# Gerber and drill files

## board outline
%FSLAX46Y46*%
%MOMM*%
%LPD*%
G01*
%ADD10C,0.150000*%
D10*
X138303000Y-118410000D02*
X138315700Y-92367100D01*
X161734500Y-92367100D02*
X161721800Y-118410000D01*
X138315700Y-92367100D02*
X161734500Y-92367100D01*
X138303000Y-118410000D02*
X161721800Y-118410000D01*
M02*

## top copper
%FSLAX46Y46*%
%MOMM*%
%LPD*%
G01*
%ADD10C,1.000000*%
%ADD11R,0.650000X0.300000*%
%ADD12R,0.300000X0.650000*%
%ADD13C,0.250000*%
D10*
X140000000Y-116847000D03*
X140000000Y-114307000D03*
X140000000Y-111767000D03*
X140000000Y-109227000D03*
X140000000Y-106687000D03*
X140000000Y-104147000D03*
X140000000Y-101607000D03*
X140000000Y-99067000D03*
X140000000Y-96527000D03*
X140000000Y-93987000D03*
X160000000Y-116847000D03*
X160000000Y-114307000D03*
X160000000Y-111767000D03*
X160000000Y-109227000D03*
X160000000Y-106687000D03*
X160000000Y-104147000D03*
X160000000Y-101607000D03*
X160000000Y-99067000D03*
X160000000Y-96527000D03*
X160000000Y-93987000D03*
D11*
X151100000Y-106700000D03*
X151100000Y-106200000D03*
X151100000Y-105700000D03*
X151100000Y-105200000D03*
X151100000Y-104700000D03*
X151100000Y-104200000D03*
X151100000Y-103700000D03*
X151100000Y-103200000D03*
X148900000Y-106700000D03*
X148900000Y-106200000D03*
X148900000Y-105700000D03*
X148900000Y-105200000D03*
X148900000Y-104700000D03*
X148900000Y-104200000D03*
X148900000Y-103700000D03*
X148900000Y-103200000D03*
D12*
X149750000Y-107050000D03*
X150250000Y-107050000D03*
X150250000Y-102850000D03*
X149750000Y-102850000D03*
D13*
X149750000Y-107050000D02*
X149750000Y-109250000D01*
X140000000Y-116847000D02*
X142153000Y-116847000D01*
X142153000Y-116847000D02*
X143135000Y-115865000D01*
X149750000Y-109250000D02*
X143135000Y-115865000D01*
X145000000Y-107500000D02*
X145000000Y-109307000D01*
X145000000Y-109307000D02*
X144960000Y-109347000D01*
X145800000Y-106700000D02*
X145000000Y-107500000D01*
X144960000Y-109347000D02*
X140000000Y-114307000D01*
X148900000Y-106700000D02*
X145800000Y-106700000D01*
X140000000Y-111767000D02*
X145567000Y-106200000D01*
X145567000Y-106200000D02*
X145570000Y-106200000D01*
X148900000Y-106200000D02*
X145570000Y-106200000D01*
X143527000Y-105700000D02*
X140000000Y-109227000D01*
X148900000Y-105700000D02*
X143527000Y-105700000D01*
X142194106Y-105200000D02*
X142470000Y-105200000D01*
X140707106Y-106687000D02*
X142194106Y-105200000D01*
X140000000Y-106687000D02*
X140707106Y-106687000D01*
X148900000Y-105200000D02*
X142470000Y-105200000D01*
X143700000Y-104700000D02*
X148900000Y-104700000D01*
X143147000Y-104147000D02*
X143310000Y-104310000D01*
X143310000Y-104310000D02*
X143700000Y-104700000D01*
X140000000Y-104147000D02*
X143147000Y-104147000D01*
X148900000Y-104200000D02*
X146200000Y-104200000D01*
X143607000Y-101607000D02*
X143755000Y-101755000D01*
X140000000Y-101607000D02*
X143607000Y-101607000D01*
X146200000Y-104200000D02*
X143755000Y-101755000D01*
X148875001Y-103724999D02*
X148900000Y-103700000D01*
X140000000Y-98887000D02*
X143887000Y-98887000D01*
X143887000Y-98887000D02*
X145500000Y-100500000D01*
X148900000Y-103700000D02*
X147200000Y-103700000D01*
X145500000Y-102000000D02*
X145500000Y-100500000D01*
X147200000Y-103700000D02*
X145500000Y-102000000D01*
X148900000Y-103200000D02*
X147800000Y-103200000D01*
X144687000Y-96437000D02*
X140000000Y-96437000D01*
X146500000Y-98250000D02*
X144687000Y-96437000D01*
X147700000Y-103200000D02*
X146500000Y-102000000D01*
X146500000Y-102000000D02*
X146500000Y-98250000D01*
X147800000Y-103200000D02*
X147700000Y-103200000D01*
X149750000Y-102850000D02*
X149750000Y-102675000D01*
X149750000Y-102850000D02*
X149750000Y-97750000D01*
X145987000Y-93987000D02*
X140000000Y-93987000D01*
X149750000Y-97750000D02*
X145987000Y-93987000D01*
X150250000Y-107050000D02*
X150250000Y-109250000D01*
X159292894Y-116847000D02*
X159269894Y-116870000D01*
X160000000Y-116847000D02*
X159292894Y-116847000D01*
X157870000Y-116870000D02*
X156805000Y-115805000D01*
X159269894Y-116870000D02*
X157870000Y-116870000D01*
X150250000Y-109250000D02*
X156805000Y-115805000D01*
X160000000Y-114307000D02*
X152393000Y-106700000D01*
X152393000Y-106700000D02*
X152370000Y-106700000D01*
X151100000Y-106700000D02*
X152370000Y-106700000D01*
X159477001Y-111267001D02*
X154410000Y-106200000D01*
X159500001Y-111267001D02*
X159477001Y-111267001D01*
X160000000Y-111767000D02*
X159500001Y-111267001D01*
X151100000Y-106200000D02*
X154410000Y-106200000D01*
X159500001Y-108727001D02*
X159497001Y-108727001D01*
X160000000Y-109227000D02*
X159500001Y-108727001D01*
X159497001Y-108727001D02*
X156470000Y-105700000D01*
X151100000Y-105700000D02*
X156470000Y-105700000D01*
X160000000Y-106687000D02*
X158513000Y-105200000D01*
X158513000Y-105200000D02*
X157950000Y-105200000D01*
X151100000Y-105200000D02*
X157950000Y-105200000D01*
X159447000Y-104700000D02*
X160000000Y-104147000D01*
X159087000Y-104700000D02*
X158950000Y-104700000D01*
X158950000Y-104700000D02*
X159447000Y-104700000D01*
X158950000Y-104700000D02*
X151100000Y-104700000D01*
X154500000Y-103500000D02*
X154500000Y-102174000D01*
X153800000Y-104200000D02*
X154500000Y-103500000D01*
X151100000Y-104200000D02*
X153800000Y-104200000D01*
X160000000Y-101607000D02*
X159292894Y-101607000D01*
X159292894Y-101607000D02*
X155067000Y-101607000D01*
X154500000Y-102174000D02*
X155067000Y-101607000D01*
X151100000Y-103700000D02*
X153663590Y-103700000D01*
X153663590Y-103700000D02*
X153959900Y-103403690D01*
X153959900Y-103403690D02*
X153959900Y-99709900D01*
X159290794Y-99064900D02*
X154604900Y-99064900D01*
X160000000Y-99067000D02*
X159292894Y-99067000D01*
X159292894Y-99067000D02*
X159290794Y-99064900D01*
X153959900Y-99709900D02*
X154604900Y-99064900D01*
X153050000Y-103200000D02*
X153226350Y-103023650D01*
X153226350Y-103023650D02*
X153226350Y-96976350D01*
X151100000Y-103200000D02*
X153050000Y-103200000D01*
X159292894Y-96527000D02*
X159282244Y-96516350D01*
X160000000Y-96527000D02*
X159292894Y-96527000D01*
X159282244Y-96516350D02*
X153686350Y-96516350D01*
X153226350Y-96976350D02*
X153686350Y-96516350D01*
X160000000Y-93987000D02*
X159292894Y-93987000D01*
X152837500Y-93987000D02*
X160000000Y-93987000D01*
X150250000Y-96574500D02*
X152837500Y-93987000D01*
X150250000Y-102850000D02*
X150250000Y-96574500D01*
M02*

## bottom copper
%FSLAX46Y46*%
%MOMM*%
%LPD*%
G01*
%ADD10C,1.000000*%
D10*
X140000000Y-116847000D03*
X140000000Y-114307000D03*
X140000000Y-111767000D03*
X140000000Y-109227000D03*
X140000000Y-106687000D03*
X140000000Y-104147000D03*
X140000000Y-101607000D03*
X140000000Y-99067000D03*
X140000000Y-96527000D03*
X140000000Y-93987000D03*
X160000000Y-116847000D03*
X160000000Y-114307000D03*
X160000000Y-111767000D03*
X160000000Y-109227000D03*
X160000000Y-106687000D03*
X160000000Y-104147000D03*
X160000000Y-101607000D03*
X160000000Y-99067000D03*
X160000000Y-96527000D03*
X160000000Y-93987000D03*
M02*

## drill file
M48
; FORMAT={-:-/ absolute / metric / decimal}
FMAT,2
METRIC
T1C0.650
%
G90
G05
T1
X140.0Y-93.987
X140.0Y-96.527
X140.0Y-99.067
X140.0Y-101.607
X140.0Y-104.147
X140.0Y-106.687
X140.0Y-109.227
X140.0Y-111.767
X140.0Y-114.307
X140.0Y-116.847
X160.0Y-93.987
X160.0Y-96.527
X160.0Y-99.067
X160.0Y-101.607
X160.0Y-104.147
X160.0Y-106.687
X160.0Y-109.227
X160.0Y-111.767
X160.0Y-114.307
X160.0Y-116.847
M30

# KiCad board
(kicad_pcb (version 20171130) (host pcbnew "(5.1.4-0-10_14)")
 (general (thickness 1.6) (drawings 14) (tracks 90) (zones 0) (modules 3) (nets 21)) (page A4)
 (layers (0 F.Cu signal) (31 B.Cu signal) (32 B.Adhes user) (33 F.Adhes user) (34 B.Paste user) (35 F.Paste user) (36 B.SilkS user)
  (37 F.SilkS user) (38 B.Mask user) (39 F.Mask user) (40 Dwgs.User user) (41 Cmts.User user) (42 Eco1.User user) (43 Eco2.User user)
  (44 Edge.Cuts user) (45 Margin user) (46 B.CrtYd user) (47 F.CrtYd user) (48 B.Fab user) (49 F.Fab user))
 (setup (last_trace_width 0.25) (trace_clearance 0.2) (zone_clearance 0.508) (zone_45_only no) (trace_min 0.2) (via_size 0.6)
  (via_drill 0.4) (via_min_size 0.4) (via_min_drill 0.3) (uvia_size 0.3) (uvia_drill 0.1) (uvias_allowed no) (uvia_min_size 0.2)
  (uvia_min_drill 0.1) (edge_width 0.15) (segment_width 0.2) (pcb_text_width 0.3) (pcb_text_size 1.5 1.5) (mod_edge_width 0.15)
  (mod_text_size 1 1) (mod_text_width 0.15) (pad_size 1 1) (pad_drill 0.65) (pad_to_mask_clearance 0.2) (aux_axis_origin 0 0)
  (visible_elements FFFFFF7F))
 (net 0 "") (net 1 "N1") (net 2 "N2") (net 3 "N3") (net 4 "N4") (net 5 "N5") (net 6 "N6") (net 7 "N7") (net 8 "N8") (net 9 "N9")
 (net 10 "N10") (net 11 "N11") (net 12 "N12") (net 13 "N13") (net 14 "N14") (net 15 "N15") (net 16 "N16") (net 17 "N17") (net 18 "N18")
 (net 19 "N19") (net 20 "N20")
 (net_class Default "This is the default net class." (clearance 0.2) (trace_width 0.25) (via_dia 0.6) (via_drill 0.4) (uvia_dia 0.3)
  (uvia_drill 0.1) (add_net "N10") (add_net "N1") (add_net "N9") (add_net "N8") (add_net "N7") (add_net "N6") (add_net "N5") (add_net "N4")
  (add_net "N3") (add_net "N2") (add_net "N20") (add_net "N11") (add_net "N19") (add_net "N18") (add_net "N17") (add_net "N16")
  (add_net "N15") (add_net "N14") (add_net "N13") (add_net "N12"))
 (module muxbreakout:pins (layer F.Cu) (at 140 105)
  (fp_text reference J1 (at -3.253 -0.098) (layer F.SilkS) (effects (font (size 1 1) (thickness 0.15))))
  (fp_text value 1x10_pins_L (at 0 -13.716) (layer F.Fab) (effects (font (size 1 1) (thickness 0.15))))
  (pad 10 thru_hole circle (at 0 11.847) (size 1 1) (drill 0.65) (layers *.Cu *.Mask) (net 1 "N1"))
  (pad 9 thru_hole circle (at 0 9.307) (size 1 1) (drill 0.65) (layers *.Cu *.Mask) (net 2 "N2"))
  (pad 8 thru_hole circle (at 0 6.767) (size 1 1) (drill 0.65) (layers *.Cu *.Mask) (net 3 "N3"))
  (pad 7 thru_hole circle (at 0 4.227) (size 1 1) (drill 0.65) (layers *.Cu *.Mask) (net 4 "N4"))
  (pad 6 thru_hole circle (at 0 1.687) (size 1 1) (drill 0.65) (layers *.Cu *.Mask) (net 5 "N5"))
  (pad 5 thru_hole circle (at 0 -0.853) (size 1 1) (drill 0.65) (layers *.Cu *.Mask) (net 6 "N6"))
  (pad 4 thru_hole circle (at 0 -3.393) (size 1 1) (drill 0.65) (layers *.Cu *.Mask) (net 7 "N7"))
  (pad 3 thru_hole circle (at 0 -5.933) (size 1 1) (drill 0.65) (layers *.Cu *.Mask) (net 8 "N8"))
  (pad 2 thru_hole circle (at 0 -8.473) (size 1 1) (drill 0.65) (layers *.Cu *.Mask) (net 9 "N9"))
  (pad 1 thru_hole circle (at 0 -11.013) (size 1 1) (drill 0.65) (layers *.Cu *.Mask) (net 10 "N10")))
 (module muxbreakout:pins (layer F.Cu) (at 160 105)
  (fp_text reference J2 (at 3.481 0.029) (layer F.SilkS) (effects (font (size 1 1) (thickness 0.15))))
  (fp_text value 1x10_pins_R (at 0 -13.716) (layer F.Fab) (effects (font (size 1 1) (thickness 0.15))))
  (pad 10 thru_hole circle (at 0 11.847) (size 1 1) (drill 0.65) (layers *.Cu *.Mask) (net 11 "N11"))
  (pad 9 thru_hole circle (at 0 9.307) (size 1 1) (drill 0.65) (layers *.Cu *.Mask) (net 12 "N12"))
  (pad 8 thru_hole circle (at 0 6.767) (size 1 1) (drill 0.65) (layers *.Cu *.Mask) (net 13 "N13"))
  (pad 7 thru_hole circle (at 0 4.227) (size 1 1) (drill 0.65) (layers *.Cu *.Mask) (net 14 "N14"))
  (pad 6 thru_hole circle (at 0 1.687) (size 1 1) (drill 0.65) (layers *.Cu *.Mask) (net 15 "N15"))
  (pad 5 thru_hole circle (at 0 -0.853) (size 1 1) (drill 0.65) (layers *.Cu *.Mask) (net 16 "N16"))
  (pad 4 thru_hole circle (at 0 -3.393) (size 1 1) (drill 0.65) (layers *.Cu *.Mask) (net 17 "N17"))
  (pad 3 thru_hole circle (at 0 -5.933) (size 1 1) (drill 0.65) (layers *.Cu *.Mask) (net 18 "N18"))
  (pad 2 thru_hole circle (at 0 -8.473) (size 1 1) (drill 0.65) (layers *.Cu *.Mask) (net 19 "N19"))
  (pad 1 thru_hole circle (at 0 -11.013) (size 1 1) (drill 0.65) (layers *.Cu *.Mask) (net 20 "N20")))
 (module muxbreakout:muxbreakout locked (layer F.Cu) (at 150 105)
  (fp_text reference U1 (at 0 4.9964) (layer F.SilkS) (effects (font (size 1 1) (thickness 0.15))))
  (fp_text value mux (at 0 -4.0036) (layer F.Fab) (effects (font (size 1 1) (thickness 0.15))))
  (pad 12 smd rect (at 1.1 1.7) (size 0.65 0.3) (layers F.Cu F.Paste F.Mask) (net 12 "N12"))
  (pad 13 smd rect (at 1.1 1.2) (size 0.65 0.3) (layers F.Cu F.Paste F.Mask) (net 13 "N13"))
  (pad 14 smd rect (at 1.1 0.7) (size 0.65 0.3) (layers F.Cu F.Paste F.Mask) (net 14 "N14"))
  (pad 15 smd rect (at 1.1 0.2) (size 0.65 0.3) (layers F.Cu F.Paste F.Mask) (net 15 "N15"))
  (pad 16 smd rect (at 1.1 -0.3) (size 0.65 0.3) (layers F.Cu F.Paste F.Mask) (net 16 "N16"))
  (pad 17 smd rect (at 1.1 -0.8) (size 0.65 0.3) (layers F.Cu F.Paste F.Mask) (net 17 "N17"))
  (pad 18 smd rect (at 1.1 -1.3) (size 0.65 0.3) (layers F.Cu F.Paste F.Mask) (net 18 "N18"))
  (pad 19 smd rect (at 1.1 -1.8) (size 0.65 0.3) (layers F.Cu F.Paste F.Mask) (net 19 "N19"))
  (pad 9 smd rect (at -1.1 1.7) (size 0.65 0.3) (layers F.Cu F.Paste F.Mask) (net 2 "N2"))
  (pad 8 smd rect (at -1.1 1.2) (size 0.65 0.3) (layers F.Cu F.Paste F.Mask) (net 3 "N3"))
  (pad 7 smd rect (at -1.1 0.7) (size 0.65 0.3) (layers F.Cu F.Paste F.Mask) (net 4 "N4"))
  (pad 6 smd rect (at -1.1 0.2) (size 0.65 0.3) (layers F.Cu F.Paste F.Mask) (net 5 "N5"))
  (pad 5 smd rect (at -1.1 -0.3) (size 0.65 0.3) (layers F.Cu F.Paste F.Mask) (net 6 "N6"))
  (pad 4 smd rect (at -1.1 -0.8) (size 0.65 0.3) (layers F.Cu F.Paste F.Mask) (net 7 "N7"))
  (pad 3 smd rect (at -1.1 -1.3) (size 0.65 0.3) (layers F.Cu F.Paste F.Mask) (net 8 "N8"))
  (pad 2 smd rect (at -1.1 -1.8) (size 0.65 0.3) (layers F.Cu F.Paste F.Mask) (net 9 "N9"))
  (pad 10 smd rect (at -0.25 2.05) (size 0.3 0.65) (layers F.Cu F.Paste F.Mask) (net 1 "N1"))
  (pad 11 smd rect (at 0.25 2.05) (size 0.3 0.65) (layers F.Cu F.Paste F.Mask) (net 11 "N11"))
  (pad 20 smd rect (at 0.25 -2.15) (size 0.3 0.65) (layers F.Cu F.Paste F.Mask) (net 20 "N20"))
  (pad 1 smd rect (at -0.25 -2.15) (size 0.3 0.65) (layers F.Cu F.Paste F.Mask) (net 10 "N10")))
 (gr_line (start 138.303 118.41) (end 138.3157 92.3671) (layer Edge.Cuts) (width 0.15))
 (gr_line (start 161.7345 92.3671) (end 161.7218 118.41) (layer Edge.Cuts) (width 0.15))
 (gr_line (start 138.3157 92.3671) (end 161.7345 92.3671) (layer Edge.Cuts) (width 0.15))
 (gr_line (start 138.303 118.41) (end 161.7218 118.41) (layer Edge.Cuts) (width 0.15))
 (segment (start 149.75 107.05) (end 149.75 109.25) (width 0.25) (layer F.Cu) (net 1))
 (segment (start 140 116.847) (end 142.153 116.847) (width 0.25) (layer F.Cu) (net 1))
 (segment (start 142.153 116.847) (end 143.135 115.865) (width 0.25) (layer F.Cu) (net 1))
 (segment (start 149.75 109.25) (end 143.135 115.865) (width 0.25) (layer F.Cu) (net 1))
 (segment (start 145 107.5) (end 145 109.307) (width 0.25) (layer F.Cu) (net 2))
 (segment (start 145 109.307) (end 144.96 109.347) (width 0.25) (layer F.Cu) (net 2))
 (segment (start 145.8 106.7) (end 145 107.5) (width 0.25) (layer F.Cu) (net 2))
 (segment (start 144.96 109.347) (end 140 114.307) (width 0.25) (layer F.Cu) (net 2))
 (segment (start 148.9 106.7) (end 145.8 106.7) (width 0.25) (layer F.Cu) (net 2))
 (segment (start 140 111.767) (end 145.567 106.2) (width 0.25) (layer F.Cu) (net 3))
 (segment (start 145.567 106.2) (end 145.57 106.2) (width 0.25) (layer F.Cu) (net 3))
 (segment (start 148.9 106.2) (end 145.57 106.2) (width 0.25) (layer F.Cu) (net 3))
 (segment (start 143.527 105.7) (end 140 109.227) (width 0.25) (layer F.Cu) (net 4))
 (segment (start 148.9 105.7) (end 143.527 105.7) (width 0.25) (layer F.Cu) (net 4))
 (segment (start 142.194106 105.2) (end 142.47 105.2) (width 0.25) (layer F.Cu) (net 5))
 (segment (start 140.707106 106.687) (end 142.194106 105.2) (width 0.25) (layer F.Cu) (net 5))
 (segment (start 140 106.687) (end 140.707106 106.687) (width 0.25) (layer F.Cu) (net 5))
 (segment (start 148.9 105.2) (end 142.47 105.2) (width 0.25) (layer F.Cu) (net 5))
 (segment (start 143.7 104.7) (end 148.9 104.7) (width 0.25) (layer F.Cu) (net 6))
 (segment (start 143.147 104.147) (end 143.31 104.31) (width 0.25) (layer F.Cu) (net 6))
 (segment (start 143.31 104.31) (end 143.7 104.7) (width 0.25) (layer F.Cu) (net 6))
 (segment (start 140 104.147) (end 143.147 104.147) (width 0.25) (layer F.Cu) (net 6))
 (segment (start 148.9 104.2) (end 146.2 104.2) (width 0.25) (layer F.Cu) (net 7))
 (segment (start 143.607 101.607) (end 143.755 101.755) (width 0.25) (layer F.Cu) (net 7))
 (segment (start 140 101.607) (end 143.607 101.607) (width 0.25) (layer F.Cu) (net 7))
 (segment (start 146.2 104.2) (end 143.755 101.755) (width 0.25) (layer F.Cu) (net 7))
 (segment (start 148.875001 103.724999) (end 148.9 103.7) (width 0.25) (layer F.Cu) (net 8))
 (segment (start 140 98.887) (end 143.887 98.887) (width 0.25) (layer F.Cu) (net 8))
 (segment (start 143.887 98.887) (end 145.5 100.5) (width 0.25) (layer F.Cu) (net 8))
 (segment (start 148.9 103.7) (end 147.2 103.7) (width 0.25) (layer F.Cu) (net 8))
 (segment (start 145.5 102) (end 145.5 100.5) (width 0.25) (layer F.Cu) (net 8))
 (segment (start 147.2 103.7) (end 145.5 102) (width 0.25) (layer F.Cu) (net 8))
 (segment (start 148.9 103.2) (end 147.8 103.2) (width 0.25) (layer F.Cu) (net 9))
 (segment (start 144.687 96.437) (end 140 96.437) (width 0.25) (layer F.Cu) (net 9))
 (segment (start 146.5 98.25) (end 144.687 96.437) (width 0.25) (layer F.Cu) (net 9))
 (segment (start 147.7 103.2) (end 146.5 102) (width 0.25) (layer F.Cu) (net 9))
 (segment (start 146.5 102) (end 146.5 98.25) (width 0.25) (layer F.Cu) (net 9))
 (segment (start 147.8 103.2) (end 147.7 103.2) (width 0.25) (layer F.Cu) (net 9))
 (segment (start 149.75 102.85) (end 149.75 102.675) (width 0.25) (layer F.Cu) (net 10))
 (segment (start 149.75 102.85) (end 149.75 97.75) (width 0.25) (layer F.Cu) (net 10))
 (segment (start 145.987 93.987) (end 140 93.987) (width 0.25) (layer F.Cu) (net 10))
 (segment (start 149.75 97.75) (end 145.987 93.987) (width 0.25) (layer F.Cu) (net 10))
 (segment (start 150.25 107.05) (end 150.25 109.25) (width 0.25) (layer F.Cu) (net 11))
 (segment (start 159.292894 116.847) (end 159.269894 116.87) (width 0.25) (layer F.Cu) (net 11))
 (segment (start 160 116.847) (end 159.292894 116.847) (width 0.25) (layer F.Cu) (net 11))
 (segment (start 157.87 116.87) (end 156.805 115.805) (width 0.25) (layer F.Cu) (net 11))
 (segment (start 159.269894 116.87) (end 157.87 116.87) (width 0.25) (layer F.Cu) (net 11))
 (segment (start 150.25 109.25) (end 156.805 115.805) (width 0.25) (layer F.Cu) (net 11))
 (segment (start 160 114.307) (end 152.393 106.7) (width 0.25) (layer F.Cu) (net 12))
 (segment (start 152.393 106.7) (end 152.37 106.7) (width 0.25) (layer F.Cu) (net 12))
 (segment (start 151.1 106.7) (end 152.37 106.7) (width 0.25) (layer F.Cu) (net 12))
 (segment (start 159.477001 111.267001) (end 154.41 106.2) (width 0.25) (layer F.Cu) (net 13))
 (segment (start 159.500001 111.267001) (end 159.477001 111.267001) (width 0.25) (layer F.Cu) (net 13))
 (segment (start 160 111.767) (end 159.500001 111.267001) (width 0.25) (layer F.Cu) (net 13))
 (segment (start 151.1 106.2) (end 154.41 106.2) (width 0.25) (layer F.Cu) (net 13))
 (segment (start 159.500001 108.727001) (end 159.497001 108.727001) (width 0.25) (layer F.Cu) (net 14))
 (segment (start 160 109.227) (end 159.500001 108.727001) (width 0.25) (layer F.Cu) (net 14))
 (segment (start 159.497001 108.727001) (end 156.47 105.7) (width 0.25) (layer F.Cu) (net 14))
 (segment (start 151.1 105.7) (end 156.47 105.7) (width 0.25) (layer F.Cu) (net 14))
 (segment (start 160 106.687) (end 158.513 105.2) (width 0.25) (layer F.Cu) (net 15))
 (segment (start 158.513 105.2) (end 157.95 105.2) (width 0.25) (layer F.Cu) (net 15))
 (segment (start 151.1 105.2) (end 157.95 105.2) (width 0.25) (layer F.Cu) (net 15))
 (segment (start 159.447 104.7) (end 160 104.147) (width 0.25) (layer F.Cu) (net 16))
 (segment (start 159.087 104.7) (end 158.95 104.7) (width 0.25) (layer F.Cu) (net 16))
 (segment (start 158.95 104.7) (end 159.447 104.7) (width 0.25) (layer F.Cu) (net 16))
 (segment (start 158.95 104.7) (end 151.1 104.7) (width 0.25) (layer F.Cu) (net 16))
 (segment (start 154.5 103.5) (end 154.5 102.174) (width 0.25) (layer F.Cu) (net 17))
 (segment (start 153.8 104.2) (end 154.5 103.5) (width 0.25) (layer F.Cu) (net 17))
 (segment (start 151.1 104.2) (end 153.8 104.2) (width 0.25) (layer F.Cu) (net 17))
 (segment (start 160 101.607) (end 159.292894 101.607) (width 0.25) (layer F.Cu) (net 17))
 (segment (start 159.292894 101.607) (end 155.067 101.607) (width 0.25) (layer F.Cu) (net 17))
 (segment (start 154.5 102.174) (end 155.067 101.607) (width 0.25) (layer F.Cu) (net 17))
 (segment (start 151.1 103.7) (end 153.66359 103.7) (width 0.25) (layer F.Cu) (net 18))
 (segment (start 153.66359 103.7) (end 153.9599 103.40369) (width 0.25) (layer F.Cu) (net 18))
 (segment (start 153.9599 103.40369) (end 153.9599 99.7099) (width 0.25) (layer F.Cu) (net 18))
 (segment (start 159.290794 99.0649) (end 154.6049 99.0649) (width 0.25) (layer F.Cu) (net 18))
 (segment (start 160 99.067) (end 159.292894 99.067) (width 0.25) (layer F.Cu) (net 18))
 (segment (start 159.292894 99.067) (end 159.290794 99.0649) (width 0.25) (layer F.Cu) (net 18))
 (segment (start 153.9599 99.7099) (end 154.6049 99.0649) (width 0.25) (layer F.Cu) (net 18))
 (segment (start 153.05 103.2) (end 153.22635 103.02365) (width 0.25) (layer F.Cu) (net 19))
 (segment (start 153.22635 103.02365) (end 153.22635 96.97635) (width 0.25) (layer F.Cu) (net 19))
 (segment (start 151.1 103.2) (end 153.05 103.2) (width 0.25) (layer F.Cu) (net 19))
 (segment (start 159.292894 96.527) (end 159.282244 96.51635) (width 0.25) (layer F.Cu) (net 19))
 (segment (start 160 96.527) (end 159.292894 96.527) (width 0.25) (layer F.Cu) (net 19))
 (segment (start 159.282244 96.51635) (end 153.68635 96.51635) (width 0.25) (layer F.Cu) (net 19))
 (segment (start 153.22635 96.97635) (end 153.68635 96.51635) (width 0.25) (layer F.Cu) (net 19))
 (segment (start 160 93.987) (end 159.292894 93.987) (width 0.25) (layer F.Cu) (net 20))
 (segment (start 152.8375 93.987) (end 160 93.987) (width 0.25) (layer F.Cu) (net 20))
 (segment (start 150.25 96.5745) (end 152.8375 93.987) (width 0.25) (layer F.Cu) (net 20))
 (segment (start 150.25 102.85) (end 150.25 96.5745) (width 0.25) (layer F.Cu) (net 20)))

